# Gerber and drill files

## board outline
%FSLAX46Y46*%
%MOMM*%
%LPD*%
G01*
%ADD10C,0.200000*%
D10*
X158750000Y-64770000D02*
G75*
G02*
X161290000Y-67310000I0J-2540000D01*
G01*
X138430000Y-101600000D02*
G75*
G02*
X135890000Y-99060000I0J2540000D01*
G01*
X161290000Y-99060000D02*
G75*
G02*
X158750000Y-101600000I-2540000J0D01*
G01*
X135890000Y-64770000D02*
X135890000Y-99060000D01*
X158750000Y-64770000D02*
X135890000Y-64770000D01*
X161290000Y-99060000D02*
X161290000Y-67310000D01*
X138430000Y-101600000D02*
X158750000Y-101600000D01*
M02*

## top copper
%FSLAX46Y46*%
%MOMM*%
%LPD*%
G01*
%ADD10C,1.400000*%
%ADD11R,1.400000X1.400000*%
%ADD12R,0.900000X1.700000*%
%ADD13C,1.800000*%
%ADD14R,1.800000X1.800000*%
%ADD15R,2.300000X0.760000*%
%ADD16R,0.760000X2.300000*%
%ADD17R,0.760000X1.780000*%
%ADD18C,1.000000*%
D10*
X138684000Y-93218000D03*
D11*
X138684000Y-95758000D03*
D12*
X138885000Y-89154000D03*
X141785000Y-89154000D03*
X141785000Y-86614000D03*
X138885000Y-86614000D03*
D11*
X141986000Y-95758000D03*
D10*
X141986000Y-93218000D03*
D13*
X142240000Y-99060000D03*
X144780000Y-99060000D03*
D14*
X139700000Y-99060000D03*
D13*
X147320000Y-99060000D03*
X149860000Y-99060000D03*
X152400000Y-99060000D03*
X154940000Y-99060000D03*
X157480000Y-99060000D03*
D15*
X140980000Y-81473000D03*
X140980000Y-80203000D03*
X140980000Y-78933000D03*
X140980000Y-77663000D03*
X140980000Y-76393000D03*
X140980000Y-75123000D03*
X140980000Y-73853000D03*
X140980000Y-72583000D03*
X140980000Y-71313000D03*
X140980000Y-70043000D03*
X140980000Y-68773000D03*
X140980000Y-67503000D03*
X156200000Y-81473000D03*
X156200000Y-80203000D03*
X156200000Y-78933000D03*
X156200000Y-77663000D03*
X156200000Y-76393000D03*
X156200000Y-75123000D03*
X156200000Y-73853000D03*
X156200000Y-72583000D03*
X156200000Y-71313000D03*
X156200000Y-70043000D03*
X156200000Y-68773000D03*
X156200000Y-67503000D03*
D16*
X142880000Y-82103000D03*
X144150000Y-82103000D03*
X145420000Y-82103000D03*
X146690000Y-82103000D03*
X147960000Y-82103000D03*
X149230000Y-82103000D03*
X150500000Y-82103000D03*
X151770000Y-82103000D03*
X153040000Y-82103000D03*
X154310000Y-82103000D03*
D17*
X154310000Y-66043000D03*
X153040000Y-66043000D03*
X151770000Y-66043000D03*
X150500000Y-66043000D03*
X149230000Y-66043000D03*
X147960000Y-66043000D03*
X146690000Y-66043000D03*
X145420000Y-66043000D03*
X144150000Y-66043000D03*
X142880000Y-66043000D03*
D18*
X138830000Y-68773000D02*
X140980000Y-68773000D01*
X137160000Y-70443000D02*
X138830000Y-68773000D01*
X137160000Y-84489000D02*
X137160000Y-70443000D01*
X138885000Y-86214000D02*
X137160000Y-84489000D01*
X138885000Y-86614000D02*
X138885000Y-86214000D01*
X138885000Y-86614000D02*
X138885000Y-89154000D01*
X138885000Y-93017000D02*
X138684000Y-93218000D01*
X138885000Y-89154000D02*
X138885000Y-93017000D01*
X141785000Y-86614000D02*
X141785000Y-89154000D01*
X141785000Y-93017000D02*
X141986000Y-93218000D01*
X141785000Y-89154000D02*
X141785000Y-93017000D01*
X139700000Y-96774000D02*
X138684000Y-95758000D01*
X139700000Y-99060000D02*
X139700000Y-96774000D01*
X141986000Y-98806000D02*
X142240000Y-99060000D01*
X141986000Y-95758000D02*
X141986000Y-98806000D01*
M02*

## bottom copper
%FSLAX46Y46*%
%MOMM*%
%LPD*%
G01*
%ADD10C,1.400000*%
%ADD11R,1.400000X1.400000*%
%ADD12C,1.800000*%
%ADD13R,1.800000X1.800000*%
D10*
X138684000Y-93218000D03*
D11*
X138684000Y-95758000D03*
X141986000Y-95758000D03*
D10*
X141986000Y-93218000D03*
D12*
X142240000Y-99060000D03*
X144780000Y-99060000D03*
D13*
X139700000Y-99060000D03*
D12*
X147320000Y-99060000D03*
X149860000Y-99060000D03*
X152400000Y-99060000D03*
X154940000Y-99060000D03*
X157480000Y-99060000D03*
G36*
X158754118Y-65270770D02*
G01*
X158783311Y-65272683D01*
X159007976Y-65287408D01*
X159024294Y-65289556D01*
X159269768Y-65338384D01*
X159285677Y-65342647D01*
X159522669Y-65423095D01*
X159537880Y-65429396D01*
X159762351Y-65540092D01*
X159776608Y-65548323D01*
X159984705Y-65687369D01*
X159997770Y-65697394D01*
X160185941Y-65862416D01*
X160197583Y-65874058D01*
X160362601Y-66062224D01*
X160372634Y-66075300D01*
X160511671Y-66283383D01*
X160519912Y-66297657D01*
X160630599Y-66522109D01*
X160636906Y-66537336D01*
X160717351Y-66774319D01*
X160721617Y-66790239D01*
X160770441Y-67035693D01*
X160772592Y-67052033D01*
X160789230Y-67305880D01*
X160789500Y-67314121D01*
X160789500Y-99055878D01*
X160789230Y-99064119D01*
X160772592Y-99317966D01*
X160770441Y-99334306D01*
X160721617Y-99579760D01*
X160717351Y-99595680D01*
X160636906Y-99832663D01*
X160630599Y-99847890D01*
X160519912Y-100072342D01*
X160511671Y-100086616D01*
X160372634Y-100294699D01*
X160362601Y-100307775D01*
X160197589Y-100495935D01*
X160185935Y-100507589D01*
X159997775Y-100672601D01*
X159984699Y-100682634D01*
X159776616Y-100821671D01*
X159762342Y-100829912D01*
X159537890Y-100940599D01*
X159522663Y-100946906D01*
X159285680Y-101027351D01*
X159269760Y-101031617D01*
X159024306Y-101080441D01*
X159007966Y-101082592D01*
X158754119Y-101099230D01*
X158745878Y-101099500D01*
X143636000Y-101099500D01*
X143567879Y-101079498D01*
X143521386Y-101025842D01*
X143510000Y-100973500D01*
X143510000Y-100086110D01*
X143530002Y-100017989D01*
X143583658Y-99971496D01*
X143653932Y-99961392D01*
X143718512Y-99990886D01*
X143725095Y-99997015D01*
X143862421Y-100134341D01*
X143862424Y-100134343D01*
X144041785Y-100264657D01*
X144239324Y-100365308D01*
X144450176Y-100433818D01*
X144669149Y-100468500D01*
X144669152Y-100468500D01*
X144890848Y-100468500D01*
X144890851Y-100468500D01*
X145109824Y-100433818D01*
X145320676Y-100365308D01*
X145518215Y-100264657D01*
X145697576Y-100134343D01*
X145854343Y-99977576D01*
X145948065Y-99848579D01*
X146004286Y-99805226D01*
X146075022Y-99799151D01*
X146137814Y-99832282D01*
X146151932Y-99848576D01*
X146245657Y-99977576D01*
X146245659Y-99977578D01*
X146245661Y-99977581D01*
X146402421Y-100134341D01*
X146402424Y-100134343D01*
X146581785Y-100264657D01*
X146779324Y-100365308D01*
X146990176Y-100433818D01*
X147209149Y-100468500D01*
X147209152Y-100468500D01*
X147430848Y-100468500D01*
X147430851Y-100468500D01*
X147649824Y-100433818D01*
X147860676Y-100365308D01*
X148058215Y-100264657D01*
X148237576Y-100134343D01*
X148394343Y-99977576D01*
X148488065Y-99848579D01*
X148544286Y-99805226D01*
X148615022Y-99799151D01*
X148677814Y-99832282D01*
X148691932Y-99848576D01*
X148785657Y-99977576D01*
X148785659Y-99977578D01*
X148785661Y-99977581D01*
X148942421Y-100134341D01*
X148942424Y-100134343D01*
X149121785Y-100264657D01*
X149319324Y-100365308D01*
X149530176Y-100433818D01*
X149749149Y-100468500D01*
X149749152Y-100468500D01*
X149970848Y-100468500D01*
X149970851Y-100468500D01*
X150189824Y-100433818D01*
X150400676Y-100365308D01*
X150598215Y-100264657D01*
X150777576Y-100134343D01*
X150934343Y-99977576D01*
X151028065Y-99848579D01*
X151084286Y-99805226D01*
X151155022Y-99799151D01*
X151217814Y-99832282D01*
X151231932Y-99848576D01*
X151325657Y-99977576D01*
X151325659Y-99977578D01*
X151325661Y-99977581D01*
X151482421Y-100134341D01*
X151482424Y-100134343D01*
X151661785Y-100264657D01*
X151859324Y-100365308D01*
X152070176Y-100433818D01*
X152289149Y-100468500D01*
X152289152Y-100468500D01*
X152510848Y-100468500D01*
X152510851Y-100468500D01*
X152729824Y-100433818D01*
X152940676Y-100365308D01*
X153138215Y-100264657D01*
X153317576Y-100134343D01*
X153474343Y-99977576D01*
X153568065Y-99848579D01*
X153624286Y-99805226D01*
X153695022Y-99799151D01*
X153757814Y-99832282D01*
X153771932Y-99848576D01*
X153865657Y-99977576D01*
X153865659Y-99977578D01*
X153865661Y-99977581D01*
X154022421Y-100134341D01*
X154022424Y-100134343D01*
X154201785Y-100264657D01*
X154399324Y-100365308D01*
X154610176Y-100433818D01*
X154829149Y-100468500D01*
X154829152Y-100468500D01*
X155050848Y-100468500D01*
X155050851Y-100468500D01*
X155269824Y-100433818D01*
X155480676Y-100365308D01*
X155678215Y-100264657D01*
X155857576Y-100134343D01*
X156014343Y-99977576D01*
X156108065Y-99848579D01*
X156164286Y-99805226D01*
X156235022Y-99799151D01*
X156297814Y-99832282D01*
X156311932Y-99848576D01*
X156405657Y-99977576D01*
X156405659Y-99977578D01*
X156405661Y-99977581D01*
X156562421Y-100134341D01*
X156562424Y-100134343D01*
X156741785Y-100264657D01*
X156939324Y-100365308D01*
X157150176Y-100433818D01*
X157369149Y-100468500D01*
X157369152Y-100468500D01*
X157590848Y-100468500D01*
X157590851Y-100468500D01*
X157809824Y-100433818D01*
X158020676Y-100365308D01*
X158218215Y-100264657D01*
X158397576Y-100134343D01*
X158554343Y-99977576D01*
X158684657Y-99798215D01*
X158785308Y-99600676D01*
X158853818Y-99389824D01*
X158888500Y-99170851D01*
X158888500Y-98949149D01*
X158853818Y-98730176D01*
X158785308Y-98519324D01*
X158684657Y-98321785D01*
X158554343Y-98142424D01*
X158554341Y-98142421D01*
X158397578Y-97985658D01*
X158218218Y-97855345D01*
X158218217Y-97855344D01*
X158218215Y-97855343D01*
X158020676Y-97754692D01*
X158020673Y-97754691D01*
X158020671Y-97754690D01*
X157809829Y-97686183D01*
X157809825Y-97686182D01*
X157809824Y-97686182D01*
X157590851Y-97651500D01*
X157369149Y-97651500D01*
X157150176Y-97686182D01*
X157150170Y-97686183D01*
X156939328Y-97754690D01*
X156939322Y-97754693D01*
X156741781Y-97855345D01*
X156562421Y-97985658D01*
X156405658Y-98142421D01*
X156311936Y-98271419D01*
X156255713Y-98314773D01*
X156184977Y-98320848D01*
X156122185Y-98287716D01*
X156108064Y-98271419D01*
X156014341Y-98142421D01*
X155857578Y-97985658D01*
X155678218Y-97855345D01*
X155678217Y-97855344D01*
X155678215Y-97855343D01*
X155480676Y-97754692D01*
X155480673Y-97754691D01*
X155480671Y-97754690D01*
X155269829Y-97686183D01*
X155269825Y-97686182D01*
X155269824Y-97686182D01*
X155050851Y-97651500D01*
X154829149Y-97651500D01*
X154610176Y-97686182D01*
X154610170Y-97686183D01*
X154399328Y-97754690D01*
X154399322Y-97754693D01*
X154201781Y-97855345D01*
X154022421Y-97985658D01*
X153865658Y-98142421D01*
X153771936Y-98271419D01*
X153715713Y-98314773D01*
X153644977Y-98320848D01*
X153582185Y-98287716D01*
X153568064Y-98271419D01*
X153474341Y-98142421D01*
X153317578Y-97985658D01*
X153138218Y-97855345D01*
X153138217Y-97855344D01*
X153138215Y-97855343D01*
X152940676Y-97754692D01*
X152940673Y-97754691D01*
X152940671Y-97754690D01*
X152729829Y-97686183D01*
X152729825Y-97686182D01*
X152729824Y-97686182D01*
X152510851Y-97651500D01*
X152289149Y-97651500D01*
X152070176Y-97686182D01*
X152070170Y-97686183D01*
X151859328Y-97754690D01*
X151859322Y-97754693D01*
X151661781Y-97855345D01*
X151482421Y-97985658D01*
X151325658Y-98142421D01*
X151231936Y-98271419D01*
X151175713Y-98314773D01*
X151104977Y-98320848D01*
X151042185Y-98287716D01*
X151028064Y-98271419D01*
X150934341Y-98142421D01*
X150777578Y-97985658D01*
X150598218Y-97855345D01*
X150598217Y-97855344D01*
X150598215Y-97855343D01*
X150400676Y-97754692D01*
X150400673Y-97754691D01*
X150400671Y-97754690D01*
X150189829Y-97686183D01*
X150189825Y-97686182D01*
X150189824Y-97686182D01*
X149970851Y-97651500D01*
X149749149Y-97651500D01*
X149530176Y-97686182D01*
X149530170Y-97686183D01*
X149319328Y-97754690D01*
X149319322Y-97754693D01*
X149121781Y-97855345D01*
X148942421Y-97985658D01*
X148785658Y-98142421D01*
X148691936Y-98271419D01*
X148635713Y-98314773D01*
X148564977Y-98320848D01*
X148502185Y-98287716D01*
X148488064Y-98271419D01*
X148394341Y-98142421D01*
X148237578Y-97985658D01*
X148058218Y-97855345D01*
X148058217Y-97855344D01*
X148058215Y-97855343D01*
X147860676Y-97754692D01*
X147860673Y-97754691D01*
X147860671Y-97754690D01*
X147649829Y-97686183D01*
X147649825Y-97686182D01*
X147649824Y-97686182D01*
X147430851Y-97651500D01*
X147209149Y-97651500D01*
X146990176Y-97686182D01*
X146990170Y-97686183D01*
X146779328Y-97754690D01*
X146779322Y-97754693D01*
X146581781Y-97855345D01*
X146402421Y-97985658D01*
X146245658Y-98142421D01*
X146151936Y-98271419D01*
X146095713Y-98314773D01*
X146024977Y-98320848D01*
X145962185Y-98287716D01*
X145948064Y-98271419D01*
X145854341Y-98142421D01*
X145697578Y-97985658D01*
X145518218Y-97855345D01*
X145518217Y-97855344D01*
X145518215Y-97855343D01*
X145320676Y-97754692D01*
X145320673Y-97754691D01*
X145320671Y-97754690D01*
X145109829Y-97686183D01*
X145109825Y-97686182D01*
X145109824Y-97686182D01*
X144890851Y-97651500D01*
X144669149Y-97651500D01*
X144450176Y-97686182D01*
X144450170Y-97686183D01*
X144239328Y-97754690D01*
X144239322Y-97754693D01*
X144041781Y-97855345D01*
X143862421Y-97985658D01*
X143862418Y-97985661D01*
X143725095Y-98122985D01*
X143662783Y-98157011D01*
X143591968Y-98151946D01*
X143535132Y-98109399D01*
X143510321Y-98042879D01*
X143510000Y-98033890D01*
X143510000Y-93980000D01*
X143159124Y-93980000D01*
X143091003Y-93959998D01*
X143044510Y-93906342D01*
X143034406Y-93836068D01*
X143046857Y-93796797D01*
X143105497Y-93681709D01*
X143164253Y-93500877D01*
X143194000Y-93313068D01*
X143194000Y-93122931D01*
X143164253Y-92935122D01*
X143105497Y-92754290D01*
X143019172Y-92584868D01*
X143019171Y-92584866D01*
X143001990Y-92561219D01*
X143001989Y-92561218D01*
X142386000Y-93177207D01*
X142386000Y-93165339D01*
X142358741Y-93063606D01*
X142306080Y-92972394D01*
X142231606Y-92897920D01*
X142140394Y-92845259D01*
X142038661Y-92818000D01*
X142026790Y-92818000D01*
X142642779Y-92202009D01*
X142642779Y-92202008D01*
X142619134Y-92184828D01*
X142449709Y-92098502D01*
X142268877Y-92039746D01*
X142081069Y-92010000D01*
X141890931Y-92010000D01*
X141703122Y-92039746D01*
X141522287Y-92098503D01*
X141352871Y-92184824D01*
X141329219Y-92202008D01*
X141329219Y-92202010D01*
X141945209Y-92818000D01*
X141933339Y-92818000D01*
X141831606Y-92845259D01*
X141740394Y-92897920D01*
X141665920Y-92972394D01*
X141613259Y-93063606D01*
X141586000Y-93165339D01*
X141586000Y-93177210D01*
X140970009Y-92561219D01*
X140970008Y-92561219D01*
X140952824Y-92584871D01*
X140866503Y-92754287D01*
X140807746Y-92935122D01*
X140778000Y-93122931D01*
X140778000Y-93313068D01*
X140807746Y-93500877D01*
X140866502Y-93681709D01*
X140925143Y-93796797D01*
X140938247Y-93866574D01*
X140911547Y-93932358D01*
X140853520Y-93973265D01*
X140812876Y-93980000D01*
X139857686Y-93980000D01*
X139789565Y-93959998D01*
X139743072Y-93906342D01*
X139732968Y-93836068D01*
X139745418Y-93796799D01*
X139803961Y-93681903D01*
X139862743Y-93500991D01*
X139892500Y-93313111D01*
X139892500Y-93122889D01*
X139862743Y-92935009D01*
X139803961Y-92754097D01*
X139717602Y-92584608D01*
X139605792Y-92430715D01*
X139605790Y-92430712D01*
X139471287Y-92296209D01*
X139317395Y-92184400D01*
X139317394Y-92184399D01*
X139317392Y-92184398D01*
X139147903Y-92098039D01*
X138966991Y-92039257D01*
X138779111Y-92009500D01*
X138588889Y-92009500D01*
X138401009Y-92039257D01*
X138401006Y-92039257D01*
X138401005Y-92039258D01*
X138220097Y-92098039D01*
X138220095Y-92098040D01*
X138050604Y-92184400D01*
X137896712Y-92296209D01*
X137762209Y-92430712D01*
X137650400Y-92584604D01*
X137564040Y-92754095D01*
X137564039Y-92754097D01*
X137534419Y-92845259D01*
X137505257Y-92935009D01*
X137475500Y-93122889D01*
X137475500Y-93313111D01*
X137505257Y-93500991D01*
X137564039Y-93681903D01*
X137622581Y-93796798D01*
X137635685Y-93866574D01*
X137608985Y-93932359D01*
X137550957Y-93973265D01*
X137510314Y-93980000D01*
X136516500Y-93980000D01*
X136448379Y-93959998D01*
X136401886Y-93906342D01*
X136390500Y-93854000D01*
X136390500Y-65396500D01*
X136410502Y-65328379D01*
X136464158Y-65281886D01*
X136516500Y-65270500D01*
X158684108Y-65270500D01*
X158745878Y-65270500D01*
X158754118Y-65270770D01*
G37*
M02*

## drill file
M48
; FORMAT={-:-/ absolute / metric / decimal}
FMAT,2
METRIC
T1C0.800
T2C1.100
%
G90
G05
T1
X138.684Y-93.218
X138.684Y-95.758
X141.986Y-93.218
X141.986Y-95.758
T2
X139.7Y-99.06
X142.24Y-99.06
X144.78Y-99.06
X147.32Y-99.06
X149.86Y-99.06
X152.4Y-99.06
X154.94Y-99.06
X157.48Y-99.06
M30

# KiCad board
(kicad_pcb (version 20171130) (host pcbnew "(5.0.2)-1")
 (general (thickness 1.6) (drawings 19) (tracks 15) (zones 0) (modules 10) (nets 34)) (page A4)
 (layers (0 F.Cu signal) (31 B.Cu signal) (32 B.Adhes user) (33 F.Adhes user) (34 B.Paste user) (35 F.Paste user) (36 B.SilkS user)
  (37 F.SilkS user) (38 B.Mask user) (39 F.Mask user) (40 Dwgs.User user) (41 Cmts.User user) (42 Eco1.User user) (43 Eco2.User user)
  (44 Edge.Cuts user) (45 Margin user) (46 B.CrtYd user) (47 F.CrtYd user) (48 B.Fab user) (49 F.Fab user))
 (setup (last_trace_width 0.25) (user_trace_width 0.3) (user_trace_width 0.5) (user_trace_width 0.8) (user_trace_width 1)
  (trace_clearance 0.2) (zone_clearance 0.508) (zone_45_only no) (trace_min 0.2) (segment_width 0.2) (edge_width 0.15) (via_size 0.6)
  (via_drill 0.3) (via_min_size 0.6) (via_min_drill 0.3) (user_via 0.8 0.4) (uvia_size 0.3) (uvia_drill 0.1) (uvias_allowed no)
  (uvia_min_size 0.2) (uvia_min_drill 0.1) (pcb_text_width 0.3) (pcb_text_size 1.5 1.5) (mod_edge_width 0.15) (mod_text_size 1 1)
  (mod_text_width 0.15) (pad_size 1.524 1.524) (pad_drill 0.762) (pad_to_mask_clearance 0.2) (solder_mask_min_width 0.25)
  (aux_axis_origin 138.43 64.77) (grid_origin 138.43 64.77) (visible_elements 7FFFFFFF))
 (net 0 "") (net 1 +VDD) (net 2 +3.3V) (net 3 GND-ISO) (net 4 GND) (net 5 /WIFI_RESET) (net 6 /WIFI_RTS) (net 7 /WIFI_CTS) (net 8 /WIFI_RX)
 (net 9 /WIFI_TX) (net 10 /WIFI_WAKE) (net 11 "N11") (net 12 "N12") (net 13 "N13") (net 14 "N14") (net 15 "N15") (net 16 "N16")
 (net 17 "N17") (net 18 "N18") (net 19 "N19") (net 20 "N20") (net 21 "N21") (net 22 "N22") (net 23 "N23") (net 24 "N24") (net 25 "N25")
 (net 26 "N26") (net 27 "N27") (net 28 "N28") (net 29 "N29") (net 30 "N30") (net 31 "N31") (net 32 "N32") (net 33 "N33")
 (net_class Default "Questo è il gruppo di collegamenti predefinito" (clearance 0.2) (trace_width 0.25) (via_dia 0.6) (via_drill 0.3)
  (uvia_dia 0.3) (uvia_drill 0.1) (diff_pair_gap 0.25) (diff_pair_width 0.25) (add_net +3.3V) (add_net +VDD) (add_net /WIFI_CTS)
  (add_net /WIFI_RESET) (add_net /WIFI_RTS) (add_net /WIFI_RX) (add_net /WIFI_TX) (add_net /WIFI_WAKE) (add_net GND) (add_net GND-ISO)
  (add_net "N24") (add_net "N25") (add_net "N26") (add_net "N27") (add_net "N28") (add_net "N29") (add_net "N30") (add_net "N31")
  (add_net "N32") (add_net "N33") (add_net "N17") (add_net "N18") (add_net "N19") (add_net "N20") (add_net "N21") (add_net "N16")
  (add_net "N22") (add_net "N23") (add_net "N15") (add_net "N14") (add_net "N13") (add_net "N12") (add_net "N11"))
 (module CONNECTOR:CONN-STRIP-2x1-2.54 (layer F.Cu) (at 138.684 94.488 90)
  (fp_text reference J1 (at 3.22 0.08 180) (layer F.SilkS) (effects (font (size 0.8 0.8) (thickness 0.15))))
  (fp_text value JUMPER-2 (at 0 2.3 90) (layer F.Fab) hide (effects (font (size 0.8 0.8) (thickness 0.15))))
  (pad 2 thru_hole circle (at 1.27 0 90) (size 1.4 1.4) (drill 0.8) (layers *.Cu *.Mask) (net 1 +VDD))
  (pad 1 thru_hole rect (at -1.27 0 90) (size 1.4 1.4) (drill 0.8) (layers *.Cu *.Mask) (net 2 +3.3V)))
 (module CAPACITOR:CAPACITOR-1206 (layer F.Cu) (at 140.335 89.154)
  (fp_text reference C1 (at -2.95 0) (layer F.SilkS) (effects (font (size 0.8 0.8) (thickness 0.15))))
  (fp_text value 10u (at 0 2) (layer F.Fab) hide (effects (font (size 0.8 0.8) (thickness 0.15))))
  (pad 1 smd rect (at -1.45 0) (size 0.9 1.7) (layers F.Cu F.Paste F.Mask) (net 1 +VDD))
  (pad 2 smd rect (at 1.45 0) (size 0.9 1.7) (layers F.Cu F.Paste F.Mask) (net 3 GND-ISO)))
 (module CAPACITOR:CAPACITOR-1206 (layer F.Cu) (at 140.335 86.614)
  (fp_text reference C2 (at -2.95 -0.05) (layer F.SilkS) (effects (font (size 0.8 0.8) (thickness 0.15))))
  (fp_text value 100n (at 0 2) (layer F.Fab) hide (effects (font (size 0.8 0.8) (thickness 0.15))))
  (pad 2 smd rect (at 1.45 0) (size 0.9 1.7) (layers F.Cu F.Paste F.Mask) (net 3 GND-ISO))
  (pad 1 smd rect (at -1.45 0) (size 0.9 1.7) (layers F.Cu F.Paste F.Mask) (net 1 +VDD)))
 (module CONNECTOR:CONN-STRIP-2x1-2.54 (layer F.Cu) (at 141.986 94.488 90)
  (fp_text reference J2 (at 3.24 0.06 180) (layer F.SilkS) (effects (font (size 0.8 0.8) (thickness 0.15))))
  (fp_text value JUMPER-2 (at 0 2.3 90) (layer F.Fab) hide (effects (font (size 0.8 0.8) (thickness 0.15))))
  (pad 1 thru_hole rect (at -1.27 0 90) (size 1.4 1.4) (drill 0.8) (layers *.Cu *.Mask) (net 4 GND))
  (pad 2 thru_hole circle (at 1.27 0 90) (size 1.4 1.4) (drill 0.8) (layers *.Cu *.Mask) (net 3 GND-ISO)))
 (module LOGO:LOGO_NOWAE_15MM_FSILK (layer F.Cu) (at 113.58 82.97)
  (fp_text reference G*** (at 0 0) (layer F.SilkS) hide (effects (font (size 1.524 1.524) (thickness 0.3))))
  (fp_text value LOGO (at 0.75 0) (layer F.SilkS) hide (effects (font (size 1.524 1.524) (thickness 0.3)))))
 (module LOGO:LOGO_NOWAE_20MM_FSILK (layer B.Cu) (at 113.48 77.57 180)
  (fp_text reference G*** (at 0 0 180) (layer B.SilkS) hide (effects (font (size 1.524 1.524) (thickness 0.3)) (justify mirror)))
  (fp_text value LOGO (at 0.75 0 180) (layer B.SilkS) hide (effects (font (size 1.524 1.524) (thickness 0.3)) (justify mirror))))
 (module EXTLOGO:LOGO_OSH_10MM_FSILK (layer B.Cu) (at 112.03 66.22 180)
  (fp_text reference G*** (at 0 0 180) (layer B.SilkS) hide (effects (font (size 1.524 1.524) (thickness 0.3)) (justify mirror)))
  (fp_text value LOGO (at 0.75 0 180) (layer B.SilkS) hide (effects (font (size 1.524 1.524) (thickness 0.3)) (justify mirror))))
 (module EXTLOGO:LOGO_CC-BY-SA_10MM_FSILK (layer B.Cu) (at 103.23 87.87 180)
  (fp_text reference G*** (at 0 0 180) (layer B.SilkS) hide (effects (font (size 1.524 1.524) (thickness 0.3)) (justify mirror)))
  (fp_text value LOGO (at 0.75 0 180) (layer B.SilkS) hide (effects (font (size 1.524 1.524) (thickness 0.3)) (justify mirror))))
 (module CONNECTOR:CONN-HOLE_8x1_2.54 (layer F.Cu) (at 148.59 99.06)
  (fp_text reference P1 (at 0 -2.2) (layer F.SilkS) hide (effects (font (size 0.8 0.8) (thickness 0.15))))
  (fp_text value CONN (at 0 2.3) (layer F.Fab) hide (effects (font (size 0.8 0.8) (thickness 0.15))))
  (pad 2 thru_hole circle (at -6.35 0) (size 1.8 1.8) (drill 1.1) (layers *.Cu *.Mask) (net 4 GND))
  (pad 3 thru_hole circle (at -3.81 0) (size 1.8 1.8) (drill 1.1) (layers *.Cu *.Mask) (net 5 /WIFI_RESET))
  (pad 1 thru_hole rect (at -8.89 0) (size 1.8 1.8) (drill 1.1) (layers *.Cu *.Mask) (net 2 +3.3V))
  (pad 4 thru_hole circle (at -1.27 0) (size 1.8 1.8) (drill 1.1) (layers *.Cu *.Mask) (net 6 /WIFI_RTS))
  (pad 5 thru_hole circle (at 1.27 0) (size 1.8 1.8) (drill 1.1) (layers *.Cu *.Mask) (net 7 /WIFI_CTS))
  (pad 6 thru_hole circle (at 3.81 0) (size 1.8 1.8) (drill 1.1) (layers *.Cu *.Mask) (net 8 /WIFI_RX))
  (pad 7 thru_hole circle (at 6.35 0) (size 1.8 1.8) (drill 1.1) (layers *.Cu *.Mask) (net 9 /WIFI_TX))
  (pad 8 thru_hole circle (at 8.89 0) (size 1.8 1.8) (drill 1.1) (layers *.Cu *.Mask) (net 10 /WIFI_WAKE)))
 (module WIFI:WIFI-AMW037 (layer F.Cu) (at 148.59 70.993)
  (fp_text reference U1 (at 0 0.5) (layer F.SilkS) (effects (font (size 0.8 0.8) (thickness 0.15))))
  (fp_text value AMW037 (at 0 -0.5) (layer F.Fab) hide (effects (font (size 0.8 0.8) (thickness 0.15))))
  (pad 12 smd rect (at -7.61 10.48) (size 2.3 0.76) (layers F.Cu F.Paste F.Mask) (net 3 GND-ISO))
  (pad 11 smd rect (at -7.61 9.21) (size 2.3 0.76) (layers F.Cu F.Paste F.Mask) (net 9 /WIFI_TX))
  (pad 10 smd rect (at -7.61 7.94) (size 2.3 0.76) (layers F.Cu F.Paste F.Mask) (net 8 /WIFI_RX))
  (pad 9 smd rect (at -7.61 6.67) (size 2.3 0.76) (layers F.Cu F.Paste F.Mask) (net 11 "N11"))
  (pad 8 smd rect (at -7.61 5.4) (size 2.3 0.76) (layers F.Cu F.Paste F.Mask) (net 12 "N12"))
  (pad 7 smd rect (at -7.61 4.13) (size 2.3 0.76) (layers F.Cu F.Paste F.Mask) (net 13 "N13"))
  (pad 6 smd rect (at -7.61 2.86) (size 2.3 0.76) (layers F.Cu F.Paste F.Mask) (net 10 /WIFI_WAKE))
  (pad 5 smd rect (at -7.61 1.59) (size 2.3 0.76) (layers F.Cu F.Paste F.Mask) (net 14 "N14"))
  (pad 4 smd rect (at -7.61 0.32) (size 2.3 0.76) (layers F.Cu F.Paste F.Mask) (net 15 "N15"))
  (pad 3 smd rect (at -7.61 -0.95) (size 2.3 0.76) (layers F.Cu F.Paste F.Mask) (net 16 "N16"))
  (pad 2 smd rect (at -7.61 -2.22) (size 2.3 0.76) (layers F.Cu F.Paste F.Mask) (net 1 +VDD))
  (pad 1 smd rect (at -7.61 -3.49) (size 2.3 0.76) (layers F.Cu F.Paste F.Mask) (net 3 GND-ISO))
  (pad 23 smd rect (at 7.61 10.48) (size 2.3 0.76) (layers F.Cu F.Paste F.Mask) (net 3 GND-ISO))
  (pad 24 smd rect (at 7.61 9.21) (size 2.3 0.76) (layers F.Cu F.Paste F.Mask) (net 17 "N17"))
  (pad 25 smd rect (at 7.61 7.94) (size 2.3 0.76) (layers F.Cu F.Paste F.Mask) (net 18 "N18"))
  (pad 26 smd rect (at 7.61 6.67) (size 2.3 0.76) (layers F.Cu F.Paste F.Mask) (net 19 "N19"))
  (pad 27 smd rect (at 7.61 5.4) (size 2.3 0.76) (layers F.Cu F.Paste F.Mask) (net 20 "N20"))
  (pad 28 smd rect (at 7.61 4.13) (size 2.3 0.76) (layers F.Cu F.Paste F.Mask) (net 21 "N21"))
  (pad 29 smd rect (at 7.61 2.86) (size 2.3 0.76) (layers F.Cu F.Paste F.Mask) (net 5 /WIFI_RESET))
  (pad 30 smd rect (at 7.61 1.59) (size 2.3 0.76) (layers F.Cu F.Paste F.Mask) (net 7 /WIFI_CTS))
  (pad 31 smd rect (at 7.61 0.32) (size 2.3 0.76) (layers F.Cu F.Paste F.Mask) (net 6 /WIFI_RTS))
  (pad 32 smd rect (at 7.61 -0.95) (size 2.3 0.76) (layers F.Cu F.Paste F.Mask) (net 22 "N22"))
  (pad 33 smd rect (at 7.61 -2.22) (size 2.3 0.76) (layers F.Cu F.Paste F.Mask) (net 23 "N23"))
  (pad 34 smd rect (at 7.61 -3.49) (size 2.3 0.76) (layers F.Cu F.Paste F.Mask) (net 3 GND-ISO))
  (pad 13 smd rect (at -5.71 11.11 90) (size 2.3 0.76) (layers F.Cu F.Paste F.Mask) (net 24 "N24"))
  (pad 14 smd rect (at -4.44 11.11 90) (size 2.3 0.76) (layers F.Cu F.Paste F.Mask) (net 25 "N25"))
  (pad 15 smd rect (at -3.17 11.11 90) (size 2.3 0.76) (layers F.Cu F.Paste F.Mask) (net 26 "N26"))
  (pad 16 smd rect (at -1.9 11.11 90) (size 2.3 0.76) (layers F.Cu F.Paste F.Mask) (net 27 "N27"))
  (pad 17 smd rect (at -0.63 11.11 90) (size 2.3 0.76) (layers F.Cu F.Paste F.Mask) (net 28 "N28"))
  (pad 18 smd rect (at 0.64 11.11 90) (size 2.3 0.76) (layers F.Cu F.Paste F.Mask) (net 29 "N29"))
  (pad 19 smd rect (at 1.91 11.11 90) (size 2.3 0.76) (layers F.Cu F.Paste F.Mask) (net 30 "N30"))
  (pad 20 smd rect (at 3.18 11.11 90) (size 2.3 0.76) (layers F.Cu F.Paste F.Mask) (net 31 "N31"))
  (pad 21 smd rect (at 4.45 11.11 90) (size 2.3 0.76) (layers F.Cu F.Paste F.Mask) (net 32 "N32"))
  (pad 22 smd rect (at 5.72 11.11 90) (size 2.3 0.76) (layers F.Cu F.Paste F.Mask) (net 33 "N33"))
  (pad 35 smd rect (at 5.72 -4.95 90) (size 1.78 0.76) (layers F.Cu F.Paste F.Mask) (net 3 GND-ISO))
  (pad 36 smd rect (at 4.45 -4.95 90) (size 1.78 0.76) (layers F.Cu F.Paste F.Mask) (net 3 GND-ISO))
  (pad 37 smd rect (at 3.18 -4.95 90) (size 1.78 0.76) (layers F.Cu F.Paste F.Mask) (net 3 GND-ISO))
  (pad 38 smd rect (at 1.91 -4.95 90) (size 1.78 0.76) (layers F.Cu F.Paste F.Mask) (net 3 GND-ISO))
  (pad 39 smd rect (at 0.64 -4.95 90) (size 1.78 0.76) (layers F.Cu F.Paste F.Mask) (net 3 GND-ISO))
  (pad 40 smd rect (at -0.63 -4.95 90) (size 1.78 0.76) (layers F.Cu F.Paste F.Mask) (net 3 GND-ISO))
  (pad 41 smd rect (at -1.9 -4.95 90) (size 1.78 0.76) (layers F.Cu F.Paste F.Mask) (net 3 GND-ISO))
  (pad 42 smd rect (at -3.17 -4.95 90) (size 1.78 0.76) (layers F.Cu F.Paste F.Mask) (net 3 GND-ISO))
  (pad 43 smd rect (at -4.44 -4.95 90) (size 1.78 0.76) (layers F.Cu F.Paste F.Mask) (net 3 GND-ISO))
  (pad 44 smd rect (at -5.71 -4.95 90) (size 1.78 0.76) (layers F.Cu F.Paste F.Mask) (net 3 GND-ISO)))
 (gr_arc (start 158.75 67.31) (end 161.29 67.31) (angle -90) (layer Edge.Cuts) (width 0.2))
 (gr_arc (start 138.43 99.06) (end 135.89 99.06) (angle -90) (layer Edge.Cuts) (width 0.2))
 (gr_arc (start 158.75 99.06) (end 158.75 101.6) (angle -90) (layer Edge.Cuts) (width 0.2))
 (gr_line (start 135.89 64.77) (end 135.89 99.06) (layer Edge.Cuts) (width 0.2))
 (gr_line (start 158.75 64.77) (end 135.89 64.77) (layer Edge.Cuts) (width 0.2))
 (gr_line (start 161.29 99.06) (end 161.29 67.31) (layer Edge.Cuts) (width 0.2))
 (gr_line (start 138.43 101.6) (end 158.75 101.6) (layer Edge.Cuts) (width 0.2))
 (segment (start 138.83 68.773) (end 140.98 68.773) (width 1) (layer F.Cu) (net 1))
 (segment (start 137.16 70.443) (end 138.83 68.773) (width 1) (layer F.Cu) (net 1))
 (segment (start 137.16 84.489) (end 137.16 70.443) (width 1) (layer F.Cu) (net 1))
 (segment (start 138.885 86.214) (end 137.16 84.489) (width 1) (layer F.Cu) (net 1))
 (segment (start 138.885 86.614) (end 138.885 86.214) (width 1) (layer F.Cu) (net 1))
 (segment (start 138.885 86.614) (end 138.885 89.154) (width 1) (layer F.Cu) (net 1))
 (segment (start 138.885 93.017) (end 138.684 93.218) (width 1) (layer F.Cu) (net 1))
 (segment (start 138.885 89.154) (end 138.885 93.017) (width 1) (layer F.Cu) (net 1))
 (segment (start 141.785 86.614) (end 141.785 89.154) (width 1) (layer F.Cu) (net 3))
 (segment (start 141.785 93.017) (end 141.986 93.218) (width 1) (layer F.Cu) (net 3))
 (segment (start 141.785 89.154) (end 141.785 93.017) (width 1) (layer F.Cu) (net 3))
 (segment (start 139.7 96.774) (end 138.684 95.758) (width 1) (layer F.Cu) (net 2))
 (segment (start 139.7 99.06) (end 139.7 96.774) (width 1) (layer F.Cu) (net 2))
 (segment (start 141.986 98.806) (end 142.24 99.06) (width 1) (layer F.Cu) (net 4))
 (segment (start 141.986 95.758) (end 141.986 98.806) (width 1) (layer F.Cu) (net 4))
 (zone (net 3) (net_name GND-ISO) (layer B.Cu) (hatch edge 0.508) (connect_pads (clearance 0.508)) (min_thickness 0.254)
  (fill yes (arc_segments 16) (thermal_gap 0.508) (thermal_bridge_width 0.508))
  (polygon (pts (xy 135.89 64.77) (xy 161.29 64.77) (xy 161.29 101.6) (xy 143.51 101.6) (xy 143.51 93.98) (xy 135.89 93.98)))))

